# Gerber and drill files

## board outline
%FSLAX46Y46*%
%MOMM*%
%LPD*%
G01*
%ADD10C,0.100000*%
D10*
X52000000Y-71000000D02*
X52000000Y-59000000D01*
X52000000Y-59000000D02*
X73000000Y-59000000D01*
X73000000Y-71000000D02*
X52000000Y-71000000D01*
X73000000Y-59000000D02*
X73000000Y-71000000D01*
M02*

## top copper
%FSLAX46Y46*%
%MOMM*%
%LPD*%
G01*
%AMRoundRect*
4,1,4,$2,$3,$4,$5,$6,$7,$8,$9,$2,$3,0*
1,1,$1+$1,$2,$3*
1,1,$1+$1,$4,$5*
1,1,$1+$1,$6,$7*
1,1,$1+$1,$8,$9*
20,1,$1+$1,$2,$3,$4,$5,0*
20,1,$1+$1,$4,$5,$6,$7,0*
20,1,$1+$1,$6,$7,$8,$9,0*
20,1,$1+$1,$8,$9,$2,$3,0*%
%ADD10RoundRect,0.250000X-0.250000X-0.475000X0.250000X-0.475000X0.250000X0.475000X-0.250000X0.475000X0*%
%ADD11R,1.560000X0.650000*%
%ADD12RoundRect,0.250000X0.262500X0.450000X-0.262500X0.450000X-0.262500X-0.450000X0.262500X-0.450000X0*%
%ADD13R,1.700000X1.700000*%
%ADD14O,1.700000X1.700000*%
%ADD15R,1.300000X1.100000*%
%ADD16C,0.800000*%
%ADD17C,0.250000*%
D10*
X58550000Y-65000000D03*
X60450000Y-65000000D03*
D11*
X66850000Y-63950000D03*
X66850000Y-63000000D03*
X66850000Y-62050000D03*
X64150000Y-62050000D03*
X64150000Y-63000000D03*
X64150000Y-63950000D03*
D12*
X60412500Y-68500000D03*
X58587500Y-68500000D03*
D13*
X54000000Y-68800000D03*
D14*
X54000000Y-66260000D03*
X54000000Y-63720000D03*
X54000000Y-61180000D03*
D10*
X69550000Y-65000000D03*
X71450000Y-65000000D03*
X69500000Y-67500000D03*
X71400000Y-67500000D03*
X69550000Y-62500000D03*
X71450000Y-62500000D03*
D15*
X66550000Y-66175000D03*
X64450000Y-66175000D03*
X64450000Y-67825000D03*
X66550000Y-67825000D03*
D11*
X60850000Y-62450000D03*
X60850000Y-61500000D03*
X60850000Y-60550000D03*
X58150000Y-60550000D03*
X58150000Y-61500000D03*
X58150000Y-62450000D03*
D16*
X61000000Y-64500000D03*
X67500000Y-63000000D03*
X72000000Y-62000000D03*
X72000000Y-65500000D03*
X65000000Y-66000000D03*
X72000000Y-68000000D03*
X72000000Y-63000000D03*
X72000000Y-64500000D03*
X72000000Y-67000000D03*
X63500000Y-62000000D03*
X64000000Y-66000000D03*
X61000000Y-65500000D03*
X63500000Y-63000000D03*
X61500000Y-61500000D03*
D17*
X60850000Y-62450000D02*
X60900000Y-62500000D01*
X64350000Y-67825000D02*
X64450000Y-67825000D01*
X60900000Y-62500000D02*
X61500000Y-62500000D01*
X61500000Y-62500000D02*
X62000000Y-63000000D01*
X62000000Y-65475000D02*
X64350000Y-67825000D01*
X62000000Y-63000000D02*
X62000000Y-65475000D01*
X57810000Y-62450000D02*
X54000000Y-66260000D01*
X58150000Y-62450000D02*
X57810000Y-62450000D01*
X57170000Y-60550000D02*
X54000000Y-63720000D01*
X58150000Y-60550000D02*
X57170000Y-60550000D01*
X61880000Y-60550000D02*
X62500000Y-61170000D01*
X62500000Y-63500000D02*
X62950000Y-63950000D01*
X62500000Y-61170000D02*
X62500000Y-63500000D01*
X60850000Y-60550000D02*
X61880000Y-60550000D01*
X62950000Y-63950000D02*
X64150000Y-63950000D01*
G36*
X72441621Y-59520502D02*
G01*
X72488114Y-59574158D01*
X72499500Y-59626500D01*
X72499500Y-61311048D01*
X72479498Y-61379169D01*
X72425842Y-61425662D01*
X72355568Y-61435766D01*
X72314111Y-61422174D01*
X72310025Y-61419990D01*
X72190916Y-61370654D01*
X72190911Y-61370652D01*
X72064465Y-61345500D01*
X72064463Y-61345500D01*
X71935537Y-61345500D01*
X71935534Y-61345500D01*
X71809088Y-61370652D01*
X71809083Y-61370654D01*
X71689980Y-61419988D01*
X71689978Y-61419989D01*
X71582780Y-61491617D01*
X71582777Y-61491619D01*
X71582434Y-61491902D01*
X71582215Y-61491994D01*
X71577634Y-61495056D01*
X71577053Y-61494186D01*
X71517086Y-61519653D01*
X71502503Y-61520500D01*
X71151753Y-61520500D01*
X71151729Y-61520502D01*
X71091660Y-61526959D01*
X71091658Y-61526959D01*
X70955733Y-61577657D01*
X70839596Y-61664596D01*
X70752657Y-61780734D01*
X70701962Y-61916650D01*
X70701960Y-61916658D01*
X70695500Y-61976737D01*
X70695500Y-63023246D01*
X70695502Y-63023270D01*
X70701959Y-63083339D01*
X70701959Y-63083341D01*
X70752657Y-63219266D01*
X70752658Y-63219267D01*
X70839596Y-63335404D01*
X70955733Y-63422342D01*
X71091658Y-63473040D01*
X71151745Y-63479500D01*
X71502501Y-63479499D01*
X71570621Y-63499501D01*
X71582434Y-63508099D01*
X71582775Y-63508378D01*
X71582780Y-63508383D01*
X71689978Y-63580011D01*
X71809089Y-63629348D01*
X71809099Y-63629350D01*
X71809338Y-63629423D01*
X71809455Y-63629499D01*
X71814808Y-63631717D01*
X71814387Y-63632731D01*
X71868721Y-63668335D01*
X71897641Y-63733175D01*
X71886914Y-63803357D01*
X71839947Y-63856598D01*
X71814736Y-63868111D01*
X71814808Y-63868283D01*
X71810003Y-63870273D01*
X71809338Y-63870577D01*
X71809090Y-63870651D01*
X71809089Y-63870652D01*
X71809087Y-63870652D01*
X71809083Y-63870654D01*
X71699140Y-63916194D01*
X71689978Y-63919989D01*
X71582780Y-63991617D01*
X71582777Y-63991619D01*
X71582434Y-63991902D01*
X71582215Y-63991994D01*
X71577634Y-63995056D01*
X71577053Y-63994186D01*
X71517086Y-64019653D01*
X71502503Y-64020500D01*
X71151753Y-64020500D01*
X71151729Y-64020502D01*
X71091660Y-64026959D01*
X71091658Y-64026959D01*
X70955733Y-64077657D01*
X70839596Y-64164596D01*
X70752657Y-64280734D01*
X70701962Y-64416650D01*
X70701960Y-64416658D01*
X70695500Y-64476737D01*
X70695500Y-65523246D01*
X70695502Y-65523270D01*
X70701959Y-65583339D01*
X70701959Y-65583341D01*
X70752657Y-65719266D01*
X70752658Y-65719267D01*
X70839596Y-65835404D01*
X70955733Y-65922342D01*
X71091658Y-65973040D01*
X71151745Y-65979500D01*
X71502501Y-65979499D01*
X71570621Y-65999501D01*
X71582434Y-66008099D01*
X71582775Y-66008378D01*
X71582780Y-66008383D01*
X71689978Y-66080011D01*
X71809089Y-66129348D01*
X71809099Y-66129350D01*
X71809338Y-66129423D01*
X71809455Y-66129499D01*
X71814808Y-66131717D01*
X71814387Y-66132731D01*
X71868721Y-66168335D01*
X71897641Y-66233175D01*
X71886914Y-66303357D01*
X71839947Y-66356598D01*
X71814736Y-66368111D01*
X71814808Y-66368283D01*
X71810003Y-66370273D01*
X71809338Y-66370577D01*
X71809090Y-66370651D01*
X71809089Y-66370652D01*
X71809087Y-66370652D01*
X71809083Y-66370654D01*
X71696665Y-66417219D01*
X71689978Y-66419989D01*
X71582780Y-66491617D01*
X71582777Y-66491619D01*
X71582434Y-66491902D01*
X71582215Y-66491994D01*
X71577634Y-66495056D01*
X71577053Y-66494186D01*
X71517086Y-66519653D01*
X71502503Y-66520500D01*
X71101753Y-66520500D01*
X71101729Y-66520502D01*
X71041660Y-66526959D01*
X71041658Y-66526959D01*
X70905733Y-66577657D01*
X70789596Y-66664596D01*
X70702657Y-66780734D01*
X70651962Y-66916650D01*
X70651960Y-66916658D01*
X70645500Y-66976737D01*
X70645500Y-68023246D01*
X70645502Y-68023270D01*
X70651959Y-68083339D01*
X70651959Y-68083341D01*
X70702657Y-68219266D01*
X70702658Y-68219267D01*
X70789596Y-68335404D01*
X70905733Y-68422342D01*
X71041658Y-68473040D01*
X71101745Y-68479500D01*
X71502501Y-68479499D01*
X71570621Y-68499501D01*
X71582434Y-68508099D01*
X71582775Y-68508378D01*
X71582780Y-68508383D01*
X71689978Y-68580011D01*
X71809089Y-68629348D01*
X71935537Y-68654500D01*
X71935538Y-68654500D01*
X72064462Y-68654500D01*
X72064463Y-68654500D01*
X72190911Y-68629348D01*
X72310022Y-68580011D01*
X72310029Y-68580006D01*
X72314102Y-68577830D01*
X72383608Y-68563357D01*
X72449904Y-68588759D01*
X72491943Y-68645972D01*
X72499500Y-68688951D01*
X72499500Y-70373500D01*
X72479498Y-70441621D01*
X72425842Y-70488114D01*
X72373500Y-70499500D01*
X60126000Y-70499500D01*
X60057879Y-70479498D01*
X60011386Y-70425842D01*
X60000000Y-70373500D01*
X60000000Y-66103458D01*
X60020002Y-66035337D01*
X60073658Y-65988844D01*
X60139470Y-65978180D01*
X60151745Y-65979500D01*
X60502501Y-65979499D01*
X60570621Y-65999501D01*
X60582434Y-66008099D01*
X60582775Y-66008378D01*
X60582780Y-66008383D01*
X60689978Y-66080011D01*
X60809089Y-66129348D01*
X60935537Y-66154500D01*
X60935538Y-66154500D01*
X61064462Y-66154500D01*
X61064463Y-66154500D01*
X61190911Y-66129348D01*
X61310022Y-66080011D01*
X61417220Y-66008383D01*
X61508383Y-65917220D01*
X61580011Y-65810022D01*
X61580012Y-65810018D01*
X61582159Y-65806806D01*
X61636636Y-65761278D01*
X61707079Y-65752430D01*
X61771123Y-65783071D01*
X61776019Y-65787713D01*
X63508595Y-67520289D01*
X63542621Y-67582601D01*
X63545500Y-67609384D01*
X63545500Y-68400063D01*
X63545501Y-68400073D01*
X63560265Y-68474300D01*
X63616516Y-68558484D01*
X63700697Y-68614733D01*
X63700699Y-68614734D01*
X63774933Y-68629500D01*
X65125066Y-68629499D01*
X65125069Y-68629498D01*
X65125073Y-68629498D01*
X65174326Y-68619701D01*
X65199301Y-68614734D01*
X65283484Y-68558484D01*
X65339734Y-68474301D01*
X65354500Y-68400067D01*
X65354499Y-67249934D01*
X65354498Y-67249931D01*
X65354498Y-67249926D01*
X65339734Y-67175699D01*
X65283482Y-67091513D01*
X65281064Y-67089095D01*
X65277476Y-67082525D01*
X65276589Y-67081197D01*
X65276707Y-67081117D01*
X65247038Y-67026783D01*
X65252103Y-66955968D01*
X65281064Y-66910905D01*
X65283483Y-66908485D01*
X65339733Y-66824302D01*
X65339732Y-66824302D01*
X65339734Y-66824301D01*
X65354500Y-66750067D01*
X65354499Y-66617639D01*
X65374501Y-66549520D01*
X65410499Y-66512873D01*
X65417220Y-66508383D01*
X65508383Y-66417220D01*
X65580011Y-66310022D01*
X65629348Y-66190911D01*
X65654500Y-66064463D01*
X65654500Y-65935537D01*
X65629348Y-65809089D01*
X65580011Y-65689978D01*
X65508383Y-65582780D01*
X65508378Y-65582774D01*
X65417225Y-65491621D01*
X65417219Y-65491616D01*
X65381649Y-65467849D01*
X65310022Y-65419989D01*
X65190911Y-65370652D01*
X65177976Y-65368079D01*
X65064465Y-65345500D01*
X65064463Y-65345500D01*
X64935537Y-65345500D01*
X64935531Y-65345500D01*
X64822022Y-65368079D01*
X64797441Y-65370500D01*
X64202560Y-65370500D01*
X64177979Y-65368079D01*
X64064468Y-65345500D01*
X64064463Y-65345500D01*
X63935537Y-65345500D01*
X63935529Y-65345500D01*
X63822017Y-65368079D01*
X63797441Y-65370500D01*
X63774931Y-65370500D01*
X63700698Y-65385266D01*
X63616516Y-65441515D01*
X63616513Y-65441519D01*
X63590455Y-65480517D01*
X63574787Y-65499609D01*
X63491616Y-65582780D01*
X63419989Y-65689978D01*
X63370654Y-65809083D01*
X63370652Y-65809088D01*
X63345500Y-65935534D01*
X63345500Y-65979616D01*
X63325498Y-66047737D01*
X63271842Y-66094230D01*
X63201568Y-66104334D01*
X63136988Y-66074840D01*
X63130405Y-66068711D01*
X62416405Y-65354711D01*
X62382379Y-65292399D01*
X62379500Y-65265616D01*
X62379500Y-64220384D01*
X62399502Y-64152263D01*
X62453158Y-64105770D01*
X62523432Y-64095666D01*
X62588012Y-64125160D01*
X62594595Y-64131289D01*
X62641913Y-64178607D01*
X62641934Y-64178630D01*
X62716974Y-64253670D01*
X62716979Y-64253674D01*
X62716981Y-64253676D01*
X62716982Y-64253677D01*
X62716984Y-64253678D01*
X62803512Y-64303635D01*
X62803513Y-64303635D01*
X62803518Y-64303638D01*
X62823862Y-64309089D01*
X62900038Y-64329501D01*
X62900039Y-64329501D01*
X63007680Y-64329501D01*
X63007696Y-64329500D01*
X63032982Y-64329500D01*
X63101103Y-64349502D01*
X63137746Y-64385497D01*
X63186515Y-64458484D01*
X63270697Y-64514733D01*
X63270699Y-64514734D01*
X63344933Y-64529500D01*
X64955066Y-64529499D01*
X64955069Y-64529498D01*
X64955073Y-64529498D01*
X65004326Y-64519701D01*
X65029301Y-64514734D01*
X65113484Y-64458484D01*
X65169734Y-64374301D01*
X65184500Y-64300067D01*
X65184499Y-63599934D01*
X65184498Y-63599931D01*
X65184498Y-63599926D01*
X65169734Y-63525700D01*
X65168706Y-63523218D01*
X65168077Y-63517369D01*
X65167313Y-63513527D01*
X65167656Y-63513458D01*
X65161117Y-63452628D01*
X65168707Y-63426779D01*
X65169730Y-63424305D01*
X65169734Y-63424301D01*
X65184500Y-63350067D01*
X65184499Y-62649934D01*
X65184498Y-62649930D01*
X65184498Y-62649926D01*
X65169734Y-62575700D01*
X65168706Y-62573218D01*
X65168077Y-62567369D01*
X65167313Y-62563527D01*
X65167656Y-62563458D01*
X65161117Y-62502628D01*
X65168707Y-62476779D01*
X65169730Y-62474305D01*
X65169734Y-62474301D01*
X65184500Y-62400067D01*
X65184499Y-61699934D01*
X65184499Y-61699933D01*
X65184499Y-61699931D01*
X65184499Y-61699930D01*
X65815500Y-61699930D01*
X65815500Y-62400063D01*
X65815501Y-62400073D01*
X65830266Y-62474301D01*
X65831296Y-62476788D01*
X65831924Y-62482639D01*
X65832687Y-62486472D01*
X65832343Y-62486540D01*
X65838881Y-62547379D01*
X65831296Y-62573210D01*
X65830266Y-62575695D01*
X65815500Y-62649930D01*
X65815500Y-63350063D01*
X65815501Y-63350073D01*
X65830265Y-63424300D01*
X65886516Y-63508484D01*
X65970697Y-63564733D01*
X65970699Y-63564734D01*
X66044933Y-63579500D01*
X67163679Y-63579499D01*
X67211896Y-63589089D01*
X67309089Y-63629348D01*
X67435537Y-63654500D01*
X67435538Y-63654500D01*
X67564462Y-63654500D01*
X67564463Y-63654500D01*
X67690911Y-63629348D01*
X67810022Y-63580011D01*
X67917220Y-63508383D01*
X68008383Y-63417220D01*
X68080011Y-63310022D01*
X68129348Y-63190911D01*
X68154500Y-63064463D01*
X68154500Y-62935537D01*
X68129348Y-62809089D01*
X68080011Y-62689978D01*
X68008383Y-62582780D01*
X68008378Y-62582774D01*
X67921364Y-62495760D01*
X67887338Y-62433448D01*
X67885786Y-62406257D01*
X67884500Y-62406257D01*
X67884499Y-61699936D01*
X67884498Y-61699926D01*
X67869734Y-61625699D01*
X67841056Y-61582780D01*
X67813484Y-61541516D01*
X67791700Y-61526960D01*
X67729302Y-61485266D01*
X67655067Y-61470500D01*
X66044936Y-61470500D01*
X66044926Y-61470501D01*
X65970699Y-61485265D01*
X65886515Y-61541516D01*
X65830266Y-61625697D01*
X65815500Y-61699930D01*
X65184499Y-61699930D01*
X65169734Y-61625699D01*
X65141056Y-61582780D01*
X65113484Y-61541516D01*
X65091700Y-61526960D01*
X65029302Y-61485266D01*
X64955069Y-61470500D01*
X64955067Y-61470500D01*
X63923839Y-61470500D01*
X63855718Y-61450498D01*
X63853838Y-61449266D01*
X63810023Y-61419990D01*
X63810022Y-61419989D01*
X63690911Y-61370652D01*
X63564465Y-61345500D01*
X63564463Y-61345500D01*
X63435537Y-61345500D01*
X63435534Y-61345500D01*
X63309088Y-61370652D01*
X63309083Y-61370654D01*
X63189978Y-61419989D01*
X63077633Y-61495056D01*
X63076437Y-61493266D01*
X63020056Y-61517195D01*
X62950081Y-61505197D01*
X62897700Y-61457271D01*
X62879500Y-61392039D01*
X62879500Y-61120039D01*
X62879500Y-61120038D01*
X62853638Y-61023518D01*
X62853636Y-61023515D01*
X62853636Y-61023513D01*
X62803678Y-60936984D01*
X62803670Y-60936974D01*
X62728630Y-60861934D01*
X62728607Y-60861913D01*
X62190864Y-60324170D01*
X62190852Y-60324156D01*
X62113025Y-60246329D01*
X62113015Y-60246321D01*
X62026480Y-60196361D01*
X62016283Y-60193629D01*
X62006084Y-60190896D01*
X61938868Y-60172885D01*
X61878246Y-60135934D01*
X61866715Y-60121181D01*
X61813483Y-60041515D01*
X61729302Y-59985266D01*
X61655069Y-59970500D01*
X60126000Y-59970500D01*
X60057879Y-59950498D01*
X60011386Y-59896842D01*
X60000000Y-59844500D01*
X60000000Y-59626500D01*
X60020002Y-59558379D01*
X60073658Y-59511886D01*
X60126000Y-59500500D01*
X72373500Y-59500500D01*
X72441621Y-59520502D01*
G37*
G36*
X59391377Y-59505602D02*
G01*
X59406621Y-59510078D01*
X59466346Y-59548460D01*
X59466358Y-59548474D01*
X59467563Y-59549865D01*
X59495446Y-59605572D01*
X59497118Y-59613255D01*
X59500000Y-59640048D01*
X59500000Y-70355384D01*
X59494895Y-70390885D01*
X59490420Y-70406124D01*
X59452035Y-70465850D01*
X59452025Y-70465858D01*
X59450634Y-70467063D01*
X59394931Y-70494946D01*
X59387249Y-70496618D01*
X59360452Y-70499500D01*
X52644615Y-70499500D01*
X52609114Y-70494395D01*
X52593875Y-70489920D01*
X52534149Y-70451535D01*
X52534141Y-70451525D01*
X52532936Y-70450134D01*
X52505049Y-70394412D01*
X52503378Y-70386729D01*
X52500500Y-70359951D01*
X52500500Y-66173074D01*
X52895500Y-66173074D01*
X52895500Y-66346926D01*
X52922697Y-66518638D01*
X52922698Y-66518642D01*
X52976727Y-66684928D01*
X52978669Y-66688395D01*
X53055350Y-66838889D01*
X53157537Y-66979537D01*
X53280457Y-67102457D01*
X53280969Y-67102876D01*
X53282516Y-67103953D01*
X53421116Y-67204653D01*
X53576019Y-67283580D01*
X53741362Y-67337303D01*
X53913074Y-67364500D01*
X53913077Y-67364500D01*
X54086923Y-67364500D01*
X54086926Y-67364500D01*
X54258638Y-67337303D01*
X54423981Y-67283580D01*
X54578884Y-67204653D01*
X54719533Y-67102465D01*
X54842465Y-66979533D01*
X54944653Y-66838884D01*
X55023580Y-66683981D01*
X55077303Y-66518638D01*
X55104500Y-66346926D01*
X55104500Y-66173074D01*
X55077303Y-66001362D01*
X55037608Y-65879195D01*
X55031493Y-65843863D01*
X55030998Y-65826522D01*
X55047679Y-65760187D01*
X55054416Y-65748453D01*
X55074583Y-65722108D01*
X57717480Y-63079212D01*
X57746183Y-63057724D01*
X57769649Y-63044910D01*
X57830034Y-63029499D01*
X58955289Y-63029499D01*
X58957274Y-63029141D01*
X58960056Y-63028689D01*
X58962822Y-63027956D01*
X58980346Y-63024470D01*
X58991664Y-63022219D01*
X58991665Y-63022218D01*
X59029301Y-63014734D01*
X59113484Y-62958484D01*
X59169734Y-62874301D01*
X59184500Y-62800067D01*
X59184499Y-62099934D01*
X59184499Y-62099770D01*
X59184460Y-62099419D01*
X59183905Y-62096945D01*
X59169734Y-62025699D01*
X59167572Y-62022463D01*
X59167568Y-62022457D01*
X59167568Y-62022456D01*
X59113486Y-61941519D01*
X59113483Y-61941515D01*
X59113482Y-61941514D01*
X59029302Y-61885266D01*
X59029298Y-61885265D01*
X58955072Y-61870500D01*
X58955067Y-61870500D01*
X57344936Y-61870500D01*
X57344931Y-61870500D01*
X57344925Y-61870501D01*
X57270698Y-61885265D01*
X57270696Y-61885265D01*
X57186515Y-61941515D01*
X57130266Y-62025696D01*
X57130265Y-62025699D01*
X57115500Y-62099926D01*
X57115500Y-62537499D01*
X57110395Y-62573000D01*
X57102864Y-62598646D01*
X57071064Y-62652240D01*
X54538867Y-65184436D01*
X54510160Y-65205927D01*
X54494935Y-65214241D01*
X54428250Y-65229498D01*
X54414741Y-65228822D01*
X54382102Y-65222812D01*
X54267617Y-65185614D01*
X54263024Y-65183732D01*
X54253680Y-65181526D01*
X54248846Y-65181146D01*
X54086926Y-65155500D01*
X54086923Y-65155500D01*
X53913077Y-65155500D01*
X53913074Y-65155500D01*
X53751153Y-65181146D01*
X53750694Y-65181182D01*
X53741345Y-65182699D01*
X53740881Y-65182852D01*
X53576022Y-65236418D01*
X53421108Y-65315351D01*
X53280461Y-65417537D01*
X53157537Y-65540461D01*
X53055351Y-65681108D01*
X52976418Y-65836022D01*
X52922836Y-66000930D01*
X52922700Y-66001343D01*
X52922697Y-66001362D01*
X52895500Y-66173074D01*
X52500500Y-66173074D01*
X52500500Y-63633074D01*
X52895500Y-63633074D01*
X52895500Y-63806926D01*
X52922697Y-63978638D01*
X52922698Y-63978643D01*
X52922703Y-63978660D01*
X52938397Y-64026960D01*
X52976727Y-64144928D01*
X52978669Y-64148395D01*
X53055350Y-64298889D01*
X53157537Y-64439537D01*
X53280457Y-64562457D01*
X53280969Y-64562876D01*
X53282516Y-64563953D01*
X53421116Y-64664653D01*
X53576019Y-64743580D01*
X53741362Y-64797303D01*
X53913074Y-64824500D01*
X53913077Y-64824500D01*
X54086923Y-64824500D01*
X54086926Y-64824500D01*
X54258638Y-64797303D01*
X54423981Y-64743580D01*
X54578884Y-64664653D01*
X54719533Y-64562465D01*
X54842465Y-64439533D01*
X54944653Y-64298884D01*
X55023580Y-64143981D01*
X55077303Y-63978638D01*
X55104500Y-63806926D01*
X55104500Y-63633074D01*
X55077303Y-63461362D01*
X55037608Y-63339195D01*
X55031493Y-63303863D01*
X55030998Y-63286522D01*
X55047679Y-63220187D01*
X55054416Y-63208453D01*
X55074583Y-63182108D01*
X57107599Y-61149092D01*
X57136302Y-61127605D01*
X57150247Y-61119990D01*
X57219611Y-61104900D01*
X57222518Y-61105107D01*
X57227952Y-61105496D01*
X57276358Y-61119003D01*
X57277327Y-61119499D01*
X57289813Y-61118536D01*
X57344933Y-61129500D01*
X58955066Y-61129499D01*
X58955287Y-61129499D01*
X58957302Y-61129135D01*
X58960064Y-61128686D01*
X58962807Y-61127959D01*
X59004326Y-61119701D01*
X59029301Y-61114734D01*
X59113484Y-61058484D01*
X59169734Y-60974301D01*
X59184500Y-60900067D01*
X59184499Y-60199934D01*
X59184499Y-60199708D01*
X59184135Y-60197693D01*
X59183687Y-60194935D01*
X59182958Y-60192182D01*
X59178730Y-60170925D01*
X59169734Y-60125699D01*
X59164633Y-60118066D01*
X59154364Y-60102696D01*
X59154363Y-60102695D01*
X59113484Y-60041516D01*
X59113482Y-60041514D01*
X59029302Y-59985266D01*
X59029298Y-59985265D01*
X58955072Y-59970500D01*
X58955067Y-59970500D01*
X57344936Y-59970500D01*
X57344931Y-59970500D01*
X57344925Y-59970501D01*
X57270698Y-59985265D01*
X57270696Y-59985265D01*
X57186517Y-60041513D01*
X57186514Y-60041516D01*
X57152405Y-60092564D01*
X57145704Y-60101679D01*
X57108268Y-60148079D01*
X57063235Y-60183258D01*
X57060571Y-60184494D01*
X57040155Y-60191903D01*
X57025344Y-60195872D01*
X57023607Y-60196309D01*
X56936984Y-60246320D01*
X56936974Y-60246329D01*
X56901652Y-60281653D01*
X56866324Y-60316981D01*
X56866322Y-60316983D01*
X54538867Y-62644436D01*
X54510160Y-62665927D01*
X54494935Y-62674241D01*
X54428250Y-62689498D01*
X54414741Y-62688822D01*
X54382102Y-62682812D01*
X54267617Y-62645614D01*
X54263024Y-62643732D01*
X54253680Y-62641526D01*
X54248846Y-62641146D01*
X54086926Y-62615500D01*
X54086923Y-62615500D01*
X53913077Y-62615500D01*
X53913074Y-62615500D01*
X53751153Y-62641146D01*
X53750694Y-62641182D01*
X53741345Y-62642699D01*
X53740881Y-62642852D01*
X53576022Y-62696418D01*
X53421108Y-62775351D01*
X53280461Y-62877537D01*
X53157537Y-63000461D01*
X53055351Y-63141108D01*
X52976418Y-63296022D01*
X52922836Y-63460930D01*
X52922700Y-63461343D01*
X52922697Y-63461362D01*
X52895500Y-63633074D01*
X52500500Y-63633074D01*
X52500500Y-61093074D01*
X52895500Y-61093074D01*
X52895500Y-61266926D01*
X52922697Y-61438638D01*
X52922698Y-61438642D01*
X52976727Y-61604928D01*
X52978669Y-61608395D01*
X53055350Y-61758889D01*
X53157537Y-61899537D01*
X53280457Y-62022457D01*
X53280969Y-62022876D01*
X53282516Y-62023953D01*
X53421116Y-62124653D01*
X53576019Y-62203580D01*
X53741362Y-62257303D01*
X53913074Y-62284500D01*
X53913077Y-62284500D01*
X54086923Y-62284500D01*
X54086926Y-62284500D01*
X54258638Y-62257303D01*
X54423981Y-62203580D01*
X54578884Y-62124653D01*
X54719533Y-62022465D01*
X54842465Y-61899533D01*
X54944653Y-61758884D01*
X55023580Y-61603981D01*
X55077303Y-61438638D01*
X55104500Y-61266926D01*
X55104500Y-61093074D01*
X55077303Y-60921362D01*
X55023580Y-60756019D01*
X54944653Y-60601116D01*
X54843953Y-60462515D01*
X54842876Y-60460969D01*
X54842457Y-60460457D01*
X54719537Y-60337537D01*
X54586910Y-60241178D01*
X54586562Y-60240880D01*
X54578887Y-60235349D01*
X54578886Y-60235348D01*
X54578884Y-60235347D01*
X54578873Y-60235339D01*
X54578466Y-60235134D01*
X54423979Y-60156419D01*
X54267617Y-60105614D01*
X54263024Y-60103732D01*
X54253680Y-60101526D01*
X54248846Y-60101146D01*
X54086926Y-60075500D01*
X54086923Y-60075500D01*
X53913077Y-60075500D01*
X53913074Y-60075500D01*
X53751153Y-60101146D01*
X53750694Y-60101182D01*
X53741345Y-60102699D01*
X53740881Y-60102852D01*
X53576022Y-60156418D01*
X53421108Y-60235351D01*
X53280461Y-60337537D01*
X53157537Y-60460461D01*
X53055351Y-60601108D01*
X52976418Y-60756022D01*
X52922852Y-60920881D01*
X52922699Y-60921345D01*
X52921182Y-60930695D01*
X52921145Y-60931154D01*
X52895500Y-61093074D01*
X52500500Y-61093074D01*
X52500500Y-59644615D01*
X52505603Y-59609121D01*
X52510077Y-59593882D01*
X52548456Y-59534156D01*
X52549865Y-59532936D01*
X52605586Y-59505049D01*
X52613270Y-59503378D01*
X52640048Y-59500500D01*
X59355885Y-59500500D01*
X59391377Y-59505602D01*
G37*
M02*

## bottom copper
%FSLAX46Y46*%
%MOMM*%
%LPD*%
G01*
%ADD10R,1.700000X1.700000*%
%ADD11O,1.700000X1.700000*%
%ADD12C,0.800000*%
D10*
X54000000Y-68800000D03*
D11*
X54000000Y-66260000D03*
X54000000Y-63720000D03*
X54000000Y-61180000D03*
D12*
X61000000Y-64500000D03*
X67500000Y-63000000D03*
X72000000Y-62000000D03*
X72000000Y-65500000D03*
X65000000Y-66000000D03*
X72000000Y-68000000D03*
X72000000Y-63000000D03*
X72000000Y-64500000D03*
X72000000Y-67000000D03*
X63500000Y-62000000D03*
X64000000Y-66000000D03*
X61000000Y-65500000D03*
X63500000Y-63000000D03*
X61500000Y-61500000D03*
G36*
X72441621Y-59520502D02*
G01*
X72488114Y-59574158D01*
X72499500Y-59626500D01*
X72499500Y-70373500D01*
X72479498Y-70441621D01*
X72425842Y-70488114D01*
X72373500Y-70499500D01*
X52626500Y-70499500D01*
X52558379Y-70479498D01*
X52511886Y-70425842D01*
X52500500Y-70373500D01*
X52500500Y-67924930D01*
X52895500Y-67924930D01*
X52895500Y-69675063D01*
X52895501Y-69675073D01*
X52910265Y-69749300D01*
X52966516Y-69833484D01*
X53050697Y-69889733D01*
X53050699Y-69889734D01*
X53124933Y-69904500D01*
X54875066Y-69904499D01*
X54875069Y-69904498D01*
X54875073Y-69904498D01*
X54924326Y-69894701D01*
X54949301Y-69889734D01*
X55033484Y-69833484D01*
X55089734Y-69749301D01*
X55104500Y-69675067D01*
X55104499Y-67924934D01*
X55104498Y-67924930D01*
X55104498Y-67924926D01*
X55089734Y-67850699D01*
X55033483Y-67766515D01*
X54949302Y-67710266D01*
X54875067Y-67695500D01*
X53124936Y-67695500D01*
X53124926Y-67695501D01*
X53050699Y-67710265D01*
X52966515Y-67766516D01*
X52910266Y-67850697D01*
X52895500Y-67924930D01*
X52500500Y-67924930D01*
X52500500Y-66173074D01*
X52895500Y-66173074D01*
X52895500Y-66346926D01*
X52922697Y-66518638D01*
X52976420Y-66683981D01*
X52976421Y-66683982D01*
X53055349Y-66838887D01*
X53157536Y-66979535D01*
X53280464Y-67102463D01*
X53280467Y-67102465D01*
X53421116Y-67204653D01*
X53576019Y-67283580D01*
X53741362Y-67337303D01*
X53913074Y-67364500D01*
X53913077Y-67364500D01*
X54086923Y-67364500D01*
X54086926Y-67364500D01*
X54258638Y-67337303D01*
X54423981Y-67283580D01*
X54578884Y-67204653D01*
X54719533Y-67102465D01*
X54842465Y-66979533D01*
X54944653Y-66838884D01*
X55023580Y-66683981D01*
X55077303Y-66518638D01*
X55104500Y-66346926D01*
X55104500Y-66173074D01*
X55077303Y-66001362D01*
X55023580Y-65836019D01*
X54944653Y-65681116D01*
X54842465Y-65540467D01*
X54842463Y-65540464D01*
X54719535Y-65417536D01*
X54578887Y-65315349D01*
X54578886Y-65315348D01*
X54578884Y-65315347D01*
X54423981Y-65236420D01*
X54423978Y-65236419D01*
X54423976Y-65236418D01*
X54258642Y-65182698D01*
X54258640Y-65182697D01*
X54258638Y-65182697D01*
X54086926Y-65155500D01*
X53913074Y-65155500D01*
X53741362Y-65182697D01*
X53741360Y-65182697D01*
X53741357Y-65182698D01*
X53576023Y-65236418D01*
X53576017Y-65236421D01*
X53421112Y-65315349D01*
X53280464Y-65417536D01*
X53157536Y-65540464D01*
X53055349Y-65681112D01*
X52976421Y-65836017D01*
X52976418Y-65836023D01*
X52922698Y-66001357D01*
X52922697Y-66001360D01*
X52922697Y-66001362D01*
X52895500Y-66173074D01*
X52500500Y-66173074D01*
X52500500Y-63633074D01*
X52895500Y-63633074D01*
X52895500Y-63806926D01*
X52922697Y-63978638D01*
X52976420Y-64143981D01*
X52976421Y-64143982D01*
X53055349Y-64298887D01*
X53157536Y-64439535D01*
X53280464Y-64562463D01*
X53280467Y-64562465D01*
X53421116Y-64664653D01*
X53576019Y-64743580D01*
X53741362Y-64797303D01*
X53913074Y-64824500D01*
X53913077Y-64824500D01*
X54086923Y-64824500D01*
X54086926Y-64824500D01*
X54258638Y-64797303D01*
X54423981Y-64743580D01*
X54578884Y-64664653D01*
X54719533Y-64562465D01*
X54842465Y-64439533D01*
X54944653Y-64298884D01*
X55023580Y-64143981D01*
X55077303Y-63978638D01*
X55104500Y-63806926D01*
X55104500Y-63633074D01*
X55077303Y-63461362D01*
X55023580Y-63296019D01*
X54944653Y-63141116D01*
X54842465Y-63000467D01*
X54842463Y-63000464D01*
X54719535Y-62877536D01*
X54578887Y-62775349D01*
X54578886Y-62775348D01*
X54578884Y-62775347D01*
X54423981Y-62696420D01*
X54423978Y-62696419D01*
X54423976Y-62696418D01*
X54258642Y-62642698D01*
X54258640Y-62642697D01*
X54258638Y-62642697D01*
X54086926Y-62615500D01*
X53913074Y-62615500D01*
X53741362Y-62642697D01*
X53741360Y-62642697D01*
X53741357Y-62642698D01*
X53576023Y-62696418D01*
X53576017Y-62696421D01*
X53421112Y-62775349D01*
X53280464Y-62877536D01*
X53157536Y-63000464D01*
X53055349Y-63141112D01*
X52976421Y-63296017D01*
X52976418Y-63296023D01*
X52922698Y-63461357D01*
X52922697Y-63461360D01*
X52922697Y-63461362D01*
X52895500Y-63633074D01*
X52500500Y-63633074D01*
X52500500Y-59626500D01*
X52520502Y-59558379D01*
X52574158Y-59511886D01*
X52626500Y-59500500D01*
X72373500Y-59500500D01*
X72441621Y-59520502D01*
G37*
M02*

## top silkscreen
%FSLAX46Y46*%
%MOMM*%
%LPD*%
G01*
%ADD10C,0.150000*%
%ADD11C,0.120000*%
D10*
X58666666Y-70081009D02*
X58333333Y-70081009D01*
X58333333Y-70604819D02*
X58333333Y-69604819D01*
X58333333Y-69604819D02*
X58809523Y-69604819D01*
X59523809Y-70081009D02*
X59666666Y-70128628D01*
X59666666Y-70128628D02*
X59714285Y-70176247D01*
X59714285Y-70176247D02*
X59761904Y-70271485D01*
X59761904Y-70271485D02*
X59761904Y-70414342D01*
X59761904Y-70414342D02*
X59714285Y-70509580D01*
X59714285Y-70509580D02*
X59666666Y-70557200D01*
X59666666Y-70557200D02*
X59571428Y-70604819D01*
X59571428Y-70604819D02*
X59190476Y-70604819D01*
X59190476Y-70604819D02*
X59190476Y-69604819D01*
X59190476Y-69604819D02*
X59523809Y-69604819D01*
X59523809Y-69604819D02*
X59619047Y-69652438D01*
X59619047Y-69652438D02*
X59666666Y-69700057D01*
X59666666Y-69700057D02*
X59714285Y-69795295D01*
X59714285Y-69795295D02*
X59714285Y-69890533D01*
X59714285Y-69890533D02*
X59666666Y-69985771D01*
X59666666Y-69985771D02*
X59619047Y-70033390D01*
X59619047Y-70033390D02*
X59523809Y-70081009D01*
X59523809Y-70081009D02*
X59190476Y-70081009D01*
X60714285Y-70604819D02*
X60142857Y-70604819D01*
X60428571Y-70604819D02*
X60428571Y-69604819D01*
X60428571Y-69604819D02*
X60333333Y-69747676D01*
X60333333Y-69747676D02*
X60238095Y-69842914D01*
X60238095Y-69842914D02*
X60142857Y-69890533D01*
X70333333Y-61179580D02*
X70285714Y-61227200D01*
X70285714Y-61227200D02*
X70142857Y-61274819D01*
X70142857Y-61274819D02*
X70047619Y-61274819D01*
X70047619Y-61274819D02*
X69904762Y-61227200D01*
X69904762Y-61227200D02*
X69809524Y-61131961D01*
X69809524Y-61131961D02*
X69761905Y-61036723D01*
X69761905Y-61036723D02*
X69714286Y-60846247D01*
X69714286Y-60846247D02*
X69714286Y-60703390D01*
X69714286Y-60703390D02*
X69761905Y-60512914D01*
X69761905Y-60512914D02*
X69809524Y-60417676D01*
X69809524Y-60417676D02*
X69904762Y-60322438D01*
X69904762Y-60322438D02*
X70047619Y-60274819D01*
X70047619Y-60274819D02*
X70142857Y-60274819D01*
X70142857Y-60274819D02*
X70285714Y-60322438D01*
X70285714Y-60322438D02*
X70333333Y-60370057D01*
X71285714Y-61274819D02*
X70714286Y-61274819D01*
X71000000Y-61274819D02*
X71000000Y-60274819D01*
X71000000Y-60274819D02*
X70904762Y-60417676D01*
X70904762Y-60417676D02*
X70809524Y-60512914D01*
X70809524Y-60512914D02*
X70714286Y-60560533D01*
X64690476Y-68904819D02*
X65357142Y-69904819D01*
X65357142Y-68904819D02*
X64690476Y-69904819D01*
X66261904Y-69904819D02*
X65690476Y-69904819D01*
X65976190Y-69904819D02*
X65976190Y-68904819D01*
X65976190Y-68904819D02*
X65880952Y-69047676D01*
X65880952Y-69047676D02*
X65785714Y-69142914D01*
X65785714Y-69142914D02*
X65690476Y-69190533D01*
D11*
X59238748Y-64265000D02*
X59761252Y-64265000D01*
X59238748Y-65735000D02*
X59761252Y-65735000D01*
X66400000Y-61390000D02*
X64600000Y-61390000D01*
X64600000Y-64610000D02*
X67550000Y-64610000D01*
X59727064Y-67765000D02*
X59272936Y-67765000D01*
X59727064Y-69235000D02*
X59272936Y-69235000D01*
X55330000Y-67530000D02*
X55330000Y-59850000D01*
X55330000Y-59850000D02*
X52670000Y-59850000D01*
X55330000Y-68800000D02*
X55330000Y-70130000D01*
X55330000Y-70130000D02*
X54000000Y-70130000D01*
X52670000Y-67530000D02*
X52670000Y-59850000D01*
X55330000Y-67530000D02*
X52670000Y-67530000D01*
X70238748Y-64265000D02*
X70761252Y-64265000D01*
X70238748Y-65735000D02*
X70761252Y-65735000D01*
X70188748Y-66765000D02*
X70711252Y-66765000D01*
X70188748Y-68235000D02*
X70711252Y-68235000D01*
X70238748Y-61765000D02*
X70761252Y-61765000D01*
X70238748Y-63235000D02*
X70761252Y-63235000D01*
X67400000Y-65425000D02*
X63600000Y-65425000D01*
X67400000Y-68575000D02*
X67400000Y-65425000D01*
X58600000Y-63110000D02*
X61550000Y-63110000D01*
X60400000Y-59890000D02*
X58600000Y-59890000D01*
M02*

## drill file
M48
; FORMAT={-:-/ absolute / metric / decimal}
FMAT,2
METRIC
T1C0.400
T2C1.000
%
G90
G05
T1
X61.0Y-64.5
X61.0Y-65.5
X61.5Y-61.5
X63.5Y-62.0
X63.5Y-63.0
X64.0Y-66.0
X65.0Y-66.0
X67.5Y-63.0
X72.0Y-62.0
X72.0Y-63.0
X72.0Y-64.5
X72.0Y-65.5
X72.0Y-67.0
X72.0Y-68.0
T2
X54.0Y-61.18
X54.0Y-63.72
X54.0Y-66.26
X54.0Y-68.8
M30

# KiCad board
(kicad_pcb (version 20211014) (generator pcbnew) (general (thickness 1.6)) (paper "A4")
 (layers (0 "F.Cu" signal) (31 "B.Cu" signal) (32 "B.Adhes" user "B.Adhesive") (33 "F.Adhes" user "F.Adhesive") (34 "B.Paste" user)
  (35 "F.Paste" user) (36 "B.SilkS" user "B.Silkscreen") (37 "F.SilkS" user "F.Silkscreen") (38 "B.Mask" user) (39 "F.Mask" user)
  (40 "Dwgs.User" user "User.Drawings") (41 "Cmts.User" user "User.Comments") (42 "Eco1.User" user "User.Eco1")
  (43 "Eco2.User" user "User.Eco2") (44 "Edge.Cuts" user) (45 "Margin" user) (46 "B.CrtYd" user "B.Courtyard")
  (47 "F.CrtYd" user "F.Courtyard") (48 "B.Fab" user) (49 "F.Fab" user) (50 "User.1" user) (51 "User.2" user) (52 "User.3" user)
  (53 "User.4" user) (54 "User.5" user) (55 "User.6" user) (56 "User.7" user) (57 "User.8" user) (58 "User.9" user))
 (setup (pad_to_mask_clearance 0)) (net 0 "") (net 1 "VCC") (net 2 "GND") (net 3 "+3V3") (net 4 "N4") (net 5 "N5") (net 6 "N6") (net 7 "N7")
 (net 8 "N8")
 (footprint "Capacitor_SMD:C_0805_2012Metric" (layer "F.Cu") (at 59.5 65)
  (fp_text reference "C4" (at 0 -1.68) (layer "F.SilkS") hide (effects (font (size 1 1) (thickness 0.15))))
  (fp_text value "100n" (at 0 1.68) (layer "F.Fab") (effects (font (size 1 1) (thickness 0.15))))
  (fp_line (start -0.261252 -0.735) (end 0.261252 -0.735) (layer "F.SilkS") (width 0.12))
  (fp_line (start -0.261252 0.735) (end 0.261252 0.735) (layer "F.SilkS") (width 0.12))
  (pad "1" smd roundrect (at -0.95 0) (size 1 1.45) (layers "F.Cu" "F.Paste" "F.Mask") (roundrect_rratio 0.25) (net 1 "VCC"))
  (pad "2" smd roundrect (at 0.95 0) (size 1 1.45) (layers "F.Cu" "F.Paste" "F.Mask") (roundrect_rratio 0.25) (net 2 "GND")))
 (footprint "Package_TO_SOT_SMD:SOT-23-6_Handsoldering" (layer "F.Cu") (at 65.5 63 180)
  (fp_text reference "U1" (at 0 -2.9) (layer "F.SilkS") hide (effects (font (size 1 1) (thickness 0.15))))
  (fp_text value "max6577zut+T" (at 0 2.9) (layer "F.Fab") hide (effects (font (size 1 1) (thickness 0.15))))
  (fp_line (start -0.9 1.61) (end 0.9 1.61) (layer "F.SilkS") (width 0.12))
  (fp_line (start 0.9 -1.61) (end -2.05 -1.61) (layer "F.SilkS") (width 0.12))
  (pad "1" smd rect (at -1.35 -0.95 180) (size 1.56 0.65) (layers "F.Cu" "F.Paste" "F.Mask") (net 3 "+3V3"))
  (pad "2" smd rect (at -1.35 0 180) (size 1.56 0.65) (layers "F.Cu" "F.Paste" "F.Mask") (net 2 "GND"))
  (pad "3" smd rect (at -1.35 0.95 180) (size 1.56 0.65) (layers "F.Cu" "F.Paste" "F.Mask") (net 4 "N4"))
  (pad "4" smd rect (at 1.35 0.95 180) (size 1.56 0.65) (layers "F.Cu" "F.Paste" "F.Mask") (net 2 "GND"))
  (pad "5" smd rect (at 1.35 0 180) (size 1.56 0.65) (layers "F.Cu" "F.Paste" "F.Mask") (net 2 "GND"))
  (pad "6" smd rect (at 1.35 -0.95 180) (size 1.56 0.65) (layers "F.Cu" "F.Paste" "F.Mask") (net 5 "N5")))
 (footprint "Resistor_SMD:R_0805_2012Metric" (layer "F.Cu") (at 59.5 68.5 180)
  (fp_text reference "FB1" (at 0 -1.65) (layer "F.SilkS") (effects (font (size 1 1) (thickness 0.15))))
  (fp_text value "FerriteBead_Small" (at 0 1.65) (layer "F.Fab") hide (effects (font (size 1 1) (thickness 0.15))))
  (fp_line (start -0.227064 0.735) (end 0.227064 0.735) (layer "F.SilkS") (width 0.12))
  (fp_line (start -0.227064 -0.735) (end 0.227064 -0.735) (layer "F.SilkS") (width 0.12))
  (pad "1" smd roundrect (at -0.9125 0 180) (size 1.025 1.4) (layers "F.Cu" "F.Paste" "F.Mask") (roundrect_rratio 0.243902) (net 3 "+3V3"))
  (pad "2" smd roundrect (at 0.9125 0 180) (size 1.025 1.4) (layers "F.Cu" "F.Paste" "F.Mask") (roundrect_rratio 0.243902) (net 1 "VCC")))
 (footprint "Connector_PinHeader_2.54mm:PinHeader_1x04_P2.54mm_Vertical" (layer "F.Cu") (at 54 68.8 180)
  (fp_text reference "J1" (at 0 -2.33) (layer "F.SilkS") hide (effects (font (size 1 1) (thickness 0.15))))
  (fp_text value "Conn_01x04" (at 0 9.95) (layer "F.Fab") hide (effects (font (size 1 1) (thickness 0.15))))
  (fp_line (start -1.33 1.27) (end -1.33 8.95) (layer "F.SilkS") (width 0.12))
  (fp_line (start -1.33 8.95) (end 1.33 8.95) (layer "F.SilkS") (width 0.12))
  (fp_line (start -1.33 0) (end -1.33 -1.33) (layer "F.SilkS") (width 0.12))
  (fp_line (start -1.33 -1.33) (end 0 -1.33) (layer "F.SilkS") (width 0.12))
  (fp_line (start 1.33 1.27) (end 1.33 8.95) (layer "F.SilkS") (width 0.12))
  (fp_line (start -1.33 1.27) (end 1.33 1.27) (layer "F.SilkS") (width 0.12))
  (pad "1" thru_hole rect (at 0 0 180) (size 1.7 1.7) (drill 1) (layers *.Cu *.Mask) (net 1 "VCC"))
  (pad "2" thru_hole oval (at 0 2.54 180) (size 1.7 1.7) (drill 1) (layers *.Cu *.Mask) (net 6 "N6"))
  (pad "3" thru_hole oval (at 0 5.08 180) (size 1.7 1.7) (drill 1) (layers *.Cu *.Mask) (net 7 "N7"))
  (pad "4" thru_hole oval (at 0 7.62 180) (size 1.7 1.7) (drill 1) (layers *.Cu *.Mask) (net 2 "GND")))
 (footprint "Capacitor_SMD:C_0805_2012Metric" (layer "F.Cu") (at 70.5 65)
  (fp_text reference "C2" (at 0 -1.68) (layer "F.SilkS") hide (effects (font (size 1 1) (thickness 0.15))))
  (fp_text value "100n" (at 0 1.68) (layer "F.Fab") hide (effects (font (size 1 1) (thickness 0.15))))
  (fp_line (start -0.261252 -0.735) (end 0.261252 -0.735) (layer "F.SilkS") (width 0.12))
  (fp_line (start -0.261252 0.735) (end 0.261252 0.735) (layer "F.SilkS") (width 0.12))
  (pad "1" smd roundrect (at -0.95 0) (size 1 1.45) (layers "F.Cu" "F.Paste" "F.Mask") (roundrect_rratio 0.25) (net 3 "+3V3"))
  (pad "2" smd roundrect (at 0.95 0) (size 1 1.45) (layers "F.Cu" "F.Paste" "F.Mask") (roundrect_rratio 0.25) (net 2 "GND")))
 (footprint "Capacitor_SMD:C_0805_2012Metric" (layer "F.Cu") (at 70.45 67.5)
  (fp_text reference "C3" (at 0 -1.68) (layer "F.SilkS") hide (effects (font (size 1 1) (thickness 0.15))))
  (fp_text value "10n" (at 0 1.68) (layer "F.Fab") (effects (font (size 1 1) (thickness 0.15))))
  (fp_line (start -0.261252 -0.735) (end 0.261252 -0.735) (layer "F.SilkS") (width 0.12))
  (fp_line (start -0.261252 0.735) (end 0.261252 0.735) (layer "F.SilkS") (width 0.12))
  (pad "1" smd roundrect (at -0.95 0) (size 1 1.45) (layers "F.Cu" "F.Paste" "F.Mask") (roundrect_rratio 0.25) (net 3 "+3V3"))
  (pad "2" smd roundrect (at 0.95 0) (size 1 1.45) (layers "F.Cu" "F.Paste" "F.Mask") (roundrect_rratio 0.25) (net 2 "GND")))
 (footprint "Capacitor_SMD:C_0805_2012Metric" (layer "F.Cu") (at 70.5 62.5)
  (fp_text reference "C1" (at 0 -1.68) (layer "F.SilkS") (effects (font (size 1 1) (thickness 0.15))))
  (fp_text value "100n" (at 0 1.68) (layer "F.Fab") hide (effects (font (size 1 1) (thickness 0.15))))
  (fp_line (start -0.261252 -0.735) (end 0.261252 -0.735) (layer "F.SilkS") (width 0.12))
  (fp_line (start -0.261252 0.735) (end 0.261252 0.735) (layer "F.SilkS") (width 0.12))
  (pad "1" smd roundrect (at -0.95 0) (size 1 1.45) (layers "F.Cu" "F.Paste" "F.Mask") (roundrect_rratio 0.25) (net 3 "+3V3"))
  (pad "2" smd roundrect (at 0.95 0) (size 1 1.45) (layers "F.Cu" "F.Paste" "F.Mask") (roundrect_rratio 0.25) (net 2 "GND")))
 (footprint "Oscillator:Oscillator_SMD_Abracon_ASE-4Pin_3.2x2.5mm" (layer "F.Cu") (at 65.5 67 180)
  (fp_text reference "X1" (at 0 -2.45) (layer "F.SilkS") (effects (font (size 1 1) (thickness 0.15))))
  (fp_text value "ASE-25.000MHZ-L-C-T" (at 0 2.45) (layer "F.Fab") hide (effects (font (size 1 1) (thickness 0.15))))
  (fp_line (start -1.9 1.575) (end 1.9 1.575) (layer "F.SilkS") (width 0.12))
  (fp_line (start -1.9 -1.575) (end -1.9 1.575) (layer "F.SilkS") (width 0.12))
  (pad "1" smd rect (at -1.05 0.825 180) (size 1.3 1.1) (layers "F.Cu" "F.Paste" "F.Mask") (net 3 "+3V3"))
  (pad "2" smd rect (at 1.05 0.825 180) (size 1.3 1.1) (layers "F.Cu" "F.Paste" "F.Mask") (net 2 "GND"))
  (pad "3" smd rect (at 1.05 -0.825 180) (size 1.3 1.1) (layers "F.Cu" "F.Paste" "F.Mask") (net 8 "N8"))
  (pad "4" smd rect (at -1.05 -0.825 180) (size 1.3 1.1) (layers "F.Cu" "F.Paste" "F.Mask") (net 3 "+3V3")))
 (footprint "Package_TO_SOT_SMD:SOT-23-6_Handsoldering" (layer "F.Cu") (at 59.5 61.5 180)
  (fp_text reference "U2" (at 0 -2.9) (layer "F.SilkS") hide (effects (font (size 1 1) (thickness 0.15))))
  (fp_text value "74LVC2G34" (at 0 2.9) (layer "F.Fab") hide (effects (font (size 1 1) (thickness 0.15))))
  (fp_line (start 0.9 -1.61) (end -2.05 -1.61) (layer "F.SilkS") (width 0.12))
  (fp_line (start -0.9 1.61) (end 0.9 1.61) (layer "F.SilkS") (width 0.12))
  (pad "1" smd rect (at -1.35 -0.95 180) (size 1.56 0.65) (layers "F.Cu" "F.Paste" "F.Mask") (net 8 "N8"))
  (pad "2" smd rect (at -1.35 0 180) (size 1.56 0.65) (layers "F.Cu" "F.Paste" "F.Mask") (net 2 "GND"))
  (pad "3" smd rect (at -1.35 0.95 180) (size 1.56 0.65) (layers "F.Cu" "F.Paste" "F.Mask") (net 5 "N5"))
  (pad "4" smd rect (at 1.35 0.95 180) (size 1.56 0.65) (layers "F.Cu" "F.Paste" "F.Mask") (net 7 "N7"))
  (pad "5" smd rect (at 1.35 0 180) (size 1.56 0.65) (layers "F.Cu" "F.Paste" "F.Mask") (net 1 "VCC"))
  (pad "6" smd rect (at 1.35 -0.95 180) (size 1.56 0.65) (layers "F.Cu" "F.Paste" "F.Mask") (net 6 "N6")))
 (gr_line (start 52 71) (end 52 59) (layer "Edge.Cuts") (width 0.1))
 (gr_line (start 52 59) (end 73 59) (layer "Edge.Cuts") (width 0.1))
 (gr_line (start 73 71) (end 52 71) (layer "Edge.Cuts") (width 0.1))
 (gr_line (start 73 59) (end 73 71) (layer "Edge.Cuts") (width 0.1))
 (via (at 61 64.5) (size 0.8) (drill 0.4) (layers "F.Cu" "B.Cu") (free) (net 2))
 (via (at 67.5 63) (size 0.8) (drill 0.4) (layers "F.Cu" "B.Cu") (free) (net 2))
 (via (at 72 62) (size 0.8) (drill 0.4) (layers "F.Cu" "B.Cu") (free) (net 2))
 (via (at 72 65.5) (size 0.8) (drill 0.4) (layers "F.Cu" "B.Cu") (free) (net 2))
 (via (at 65 66) (size 0.8) (drill 0.4) (layers "F.Cu" "B.Cu") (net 2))
 (via (at 72 68) (size 0.8) (drill 0.4) (layers "F.Cu" "B.Cu") (free) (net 2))
 (via (at 72 63) (size 0.8) (drill 0.4) (layers "F.Cu" "B.Cu") (free) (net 2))
 (via (at 72 64.5) (size 0.8) (drill 0.4) (layers "F.Cu" "B.Cu") (free) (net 2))
 (via (at 72 67) (size 0.8) (drill 0.4) (layers "F.Cu" "B.Cu") (free) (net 2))
 (via (at 63.5 62) (size 0.8) (drill 0.4) (layers "F.Cu" "B.Cu") (free) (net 2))
 (via (at 64 66) (size 0.8) (drill 0.4) (layers "F.Cu" "B.Cu") (free) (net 2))
 (via (at 61 65.5) (size 0.8) (drill 0.4) (layers "F.Cu" "B.Cu") (free) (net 2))
 (via (at 63.5 63) (size 0.8) (drill 0.4) (layers "F.Cu" "B.Cu") (free) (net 2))
 (via (at 61.5 61.5) (size 0.8) (drill 0.4) (layers "F.Cu" "B.Cu") (free) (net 2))
 (segment (start 60.85 62.45) (end 60.9 62.5) (width 0.25) (layer "F.Cu") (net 8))
 (segment (start 64.35 67.825) (end 64.45 67.825) (width 0.25) (layer "F.Cu") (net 8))
 (segment (start 60.9 62.5) (end 61.5 62.5) (width 0.25) (layer "F.Cu") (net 8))
 (segment (start 61.5 62.5) (end 62 63) (width 0.25) (layer "F.Cu") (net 8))
 (segment (start 62 65.475) (end 64.35 67.825) (width 0.25) (layer "F.Cu") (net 8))
 (segment (start 62 63) (end 62 65.475) (width 0.25) (layer "F.Cu") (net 8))
 (segment (start 57.81 62.45) (end 54 66.26) (width 0.25) (layer "F.Cu") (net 6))
 (segment (start 58.15 62.45) (end 57.81 62.45) (width 0.25) (layer "F.Cu") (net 6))
 (segment (start 57.17 60.55) (end 54 63.72) (width 0.25) (layer "F.Cu") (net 7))
 (segment (start 58.15 60.55) (end 57.17 60.55) (width 0.25) (layer "F.Cu") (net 7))
 (segment (start 61.88 60.55) (end 62.5 61.17) (width 0.25) (layer "F.Cu") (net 5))
 (segment (start 62.5 63.5) (end 62.95 63.95) (width 0.25) (layer "F.Cu") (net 5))
 (segment (start 62.5 61.17) (end 62.5 63.5) (width 0.25) (layer "F.Cu") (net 5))
 (segment (start 60.85 60.55) (end 61.88 60.55) (width 0.25) (layer "F.Cu") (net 5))
 (segment (start 62.95 63.95) (end 64.15 63.95) (width 0.25) (layer "F.Cu") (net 5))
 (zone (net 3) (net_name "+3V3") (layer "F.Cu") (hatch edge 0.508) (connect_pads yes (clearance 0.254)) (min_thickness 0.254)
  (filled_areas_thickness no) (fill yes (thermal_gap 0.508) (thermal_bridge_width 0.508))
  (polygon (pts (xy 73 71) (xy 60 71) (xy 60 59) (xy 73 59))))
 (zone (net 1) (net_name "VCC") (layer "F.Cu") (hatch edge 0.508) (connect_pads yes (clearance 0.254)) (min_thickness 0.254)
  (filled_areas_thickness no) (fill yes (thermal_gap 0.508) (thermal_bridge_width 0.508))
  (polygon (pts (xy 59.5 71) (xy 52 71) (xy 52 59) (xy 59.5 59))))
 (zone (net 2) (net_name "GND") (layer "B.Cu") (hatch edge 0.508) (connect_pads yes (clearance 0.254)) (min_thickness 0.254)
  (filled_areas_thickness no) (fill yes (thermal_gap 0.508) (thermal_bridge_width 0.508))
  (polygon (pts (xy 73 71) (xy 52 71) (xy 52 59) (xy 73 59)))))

